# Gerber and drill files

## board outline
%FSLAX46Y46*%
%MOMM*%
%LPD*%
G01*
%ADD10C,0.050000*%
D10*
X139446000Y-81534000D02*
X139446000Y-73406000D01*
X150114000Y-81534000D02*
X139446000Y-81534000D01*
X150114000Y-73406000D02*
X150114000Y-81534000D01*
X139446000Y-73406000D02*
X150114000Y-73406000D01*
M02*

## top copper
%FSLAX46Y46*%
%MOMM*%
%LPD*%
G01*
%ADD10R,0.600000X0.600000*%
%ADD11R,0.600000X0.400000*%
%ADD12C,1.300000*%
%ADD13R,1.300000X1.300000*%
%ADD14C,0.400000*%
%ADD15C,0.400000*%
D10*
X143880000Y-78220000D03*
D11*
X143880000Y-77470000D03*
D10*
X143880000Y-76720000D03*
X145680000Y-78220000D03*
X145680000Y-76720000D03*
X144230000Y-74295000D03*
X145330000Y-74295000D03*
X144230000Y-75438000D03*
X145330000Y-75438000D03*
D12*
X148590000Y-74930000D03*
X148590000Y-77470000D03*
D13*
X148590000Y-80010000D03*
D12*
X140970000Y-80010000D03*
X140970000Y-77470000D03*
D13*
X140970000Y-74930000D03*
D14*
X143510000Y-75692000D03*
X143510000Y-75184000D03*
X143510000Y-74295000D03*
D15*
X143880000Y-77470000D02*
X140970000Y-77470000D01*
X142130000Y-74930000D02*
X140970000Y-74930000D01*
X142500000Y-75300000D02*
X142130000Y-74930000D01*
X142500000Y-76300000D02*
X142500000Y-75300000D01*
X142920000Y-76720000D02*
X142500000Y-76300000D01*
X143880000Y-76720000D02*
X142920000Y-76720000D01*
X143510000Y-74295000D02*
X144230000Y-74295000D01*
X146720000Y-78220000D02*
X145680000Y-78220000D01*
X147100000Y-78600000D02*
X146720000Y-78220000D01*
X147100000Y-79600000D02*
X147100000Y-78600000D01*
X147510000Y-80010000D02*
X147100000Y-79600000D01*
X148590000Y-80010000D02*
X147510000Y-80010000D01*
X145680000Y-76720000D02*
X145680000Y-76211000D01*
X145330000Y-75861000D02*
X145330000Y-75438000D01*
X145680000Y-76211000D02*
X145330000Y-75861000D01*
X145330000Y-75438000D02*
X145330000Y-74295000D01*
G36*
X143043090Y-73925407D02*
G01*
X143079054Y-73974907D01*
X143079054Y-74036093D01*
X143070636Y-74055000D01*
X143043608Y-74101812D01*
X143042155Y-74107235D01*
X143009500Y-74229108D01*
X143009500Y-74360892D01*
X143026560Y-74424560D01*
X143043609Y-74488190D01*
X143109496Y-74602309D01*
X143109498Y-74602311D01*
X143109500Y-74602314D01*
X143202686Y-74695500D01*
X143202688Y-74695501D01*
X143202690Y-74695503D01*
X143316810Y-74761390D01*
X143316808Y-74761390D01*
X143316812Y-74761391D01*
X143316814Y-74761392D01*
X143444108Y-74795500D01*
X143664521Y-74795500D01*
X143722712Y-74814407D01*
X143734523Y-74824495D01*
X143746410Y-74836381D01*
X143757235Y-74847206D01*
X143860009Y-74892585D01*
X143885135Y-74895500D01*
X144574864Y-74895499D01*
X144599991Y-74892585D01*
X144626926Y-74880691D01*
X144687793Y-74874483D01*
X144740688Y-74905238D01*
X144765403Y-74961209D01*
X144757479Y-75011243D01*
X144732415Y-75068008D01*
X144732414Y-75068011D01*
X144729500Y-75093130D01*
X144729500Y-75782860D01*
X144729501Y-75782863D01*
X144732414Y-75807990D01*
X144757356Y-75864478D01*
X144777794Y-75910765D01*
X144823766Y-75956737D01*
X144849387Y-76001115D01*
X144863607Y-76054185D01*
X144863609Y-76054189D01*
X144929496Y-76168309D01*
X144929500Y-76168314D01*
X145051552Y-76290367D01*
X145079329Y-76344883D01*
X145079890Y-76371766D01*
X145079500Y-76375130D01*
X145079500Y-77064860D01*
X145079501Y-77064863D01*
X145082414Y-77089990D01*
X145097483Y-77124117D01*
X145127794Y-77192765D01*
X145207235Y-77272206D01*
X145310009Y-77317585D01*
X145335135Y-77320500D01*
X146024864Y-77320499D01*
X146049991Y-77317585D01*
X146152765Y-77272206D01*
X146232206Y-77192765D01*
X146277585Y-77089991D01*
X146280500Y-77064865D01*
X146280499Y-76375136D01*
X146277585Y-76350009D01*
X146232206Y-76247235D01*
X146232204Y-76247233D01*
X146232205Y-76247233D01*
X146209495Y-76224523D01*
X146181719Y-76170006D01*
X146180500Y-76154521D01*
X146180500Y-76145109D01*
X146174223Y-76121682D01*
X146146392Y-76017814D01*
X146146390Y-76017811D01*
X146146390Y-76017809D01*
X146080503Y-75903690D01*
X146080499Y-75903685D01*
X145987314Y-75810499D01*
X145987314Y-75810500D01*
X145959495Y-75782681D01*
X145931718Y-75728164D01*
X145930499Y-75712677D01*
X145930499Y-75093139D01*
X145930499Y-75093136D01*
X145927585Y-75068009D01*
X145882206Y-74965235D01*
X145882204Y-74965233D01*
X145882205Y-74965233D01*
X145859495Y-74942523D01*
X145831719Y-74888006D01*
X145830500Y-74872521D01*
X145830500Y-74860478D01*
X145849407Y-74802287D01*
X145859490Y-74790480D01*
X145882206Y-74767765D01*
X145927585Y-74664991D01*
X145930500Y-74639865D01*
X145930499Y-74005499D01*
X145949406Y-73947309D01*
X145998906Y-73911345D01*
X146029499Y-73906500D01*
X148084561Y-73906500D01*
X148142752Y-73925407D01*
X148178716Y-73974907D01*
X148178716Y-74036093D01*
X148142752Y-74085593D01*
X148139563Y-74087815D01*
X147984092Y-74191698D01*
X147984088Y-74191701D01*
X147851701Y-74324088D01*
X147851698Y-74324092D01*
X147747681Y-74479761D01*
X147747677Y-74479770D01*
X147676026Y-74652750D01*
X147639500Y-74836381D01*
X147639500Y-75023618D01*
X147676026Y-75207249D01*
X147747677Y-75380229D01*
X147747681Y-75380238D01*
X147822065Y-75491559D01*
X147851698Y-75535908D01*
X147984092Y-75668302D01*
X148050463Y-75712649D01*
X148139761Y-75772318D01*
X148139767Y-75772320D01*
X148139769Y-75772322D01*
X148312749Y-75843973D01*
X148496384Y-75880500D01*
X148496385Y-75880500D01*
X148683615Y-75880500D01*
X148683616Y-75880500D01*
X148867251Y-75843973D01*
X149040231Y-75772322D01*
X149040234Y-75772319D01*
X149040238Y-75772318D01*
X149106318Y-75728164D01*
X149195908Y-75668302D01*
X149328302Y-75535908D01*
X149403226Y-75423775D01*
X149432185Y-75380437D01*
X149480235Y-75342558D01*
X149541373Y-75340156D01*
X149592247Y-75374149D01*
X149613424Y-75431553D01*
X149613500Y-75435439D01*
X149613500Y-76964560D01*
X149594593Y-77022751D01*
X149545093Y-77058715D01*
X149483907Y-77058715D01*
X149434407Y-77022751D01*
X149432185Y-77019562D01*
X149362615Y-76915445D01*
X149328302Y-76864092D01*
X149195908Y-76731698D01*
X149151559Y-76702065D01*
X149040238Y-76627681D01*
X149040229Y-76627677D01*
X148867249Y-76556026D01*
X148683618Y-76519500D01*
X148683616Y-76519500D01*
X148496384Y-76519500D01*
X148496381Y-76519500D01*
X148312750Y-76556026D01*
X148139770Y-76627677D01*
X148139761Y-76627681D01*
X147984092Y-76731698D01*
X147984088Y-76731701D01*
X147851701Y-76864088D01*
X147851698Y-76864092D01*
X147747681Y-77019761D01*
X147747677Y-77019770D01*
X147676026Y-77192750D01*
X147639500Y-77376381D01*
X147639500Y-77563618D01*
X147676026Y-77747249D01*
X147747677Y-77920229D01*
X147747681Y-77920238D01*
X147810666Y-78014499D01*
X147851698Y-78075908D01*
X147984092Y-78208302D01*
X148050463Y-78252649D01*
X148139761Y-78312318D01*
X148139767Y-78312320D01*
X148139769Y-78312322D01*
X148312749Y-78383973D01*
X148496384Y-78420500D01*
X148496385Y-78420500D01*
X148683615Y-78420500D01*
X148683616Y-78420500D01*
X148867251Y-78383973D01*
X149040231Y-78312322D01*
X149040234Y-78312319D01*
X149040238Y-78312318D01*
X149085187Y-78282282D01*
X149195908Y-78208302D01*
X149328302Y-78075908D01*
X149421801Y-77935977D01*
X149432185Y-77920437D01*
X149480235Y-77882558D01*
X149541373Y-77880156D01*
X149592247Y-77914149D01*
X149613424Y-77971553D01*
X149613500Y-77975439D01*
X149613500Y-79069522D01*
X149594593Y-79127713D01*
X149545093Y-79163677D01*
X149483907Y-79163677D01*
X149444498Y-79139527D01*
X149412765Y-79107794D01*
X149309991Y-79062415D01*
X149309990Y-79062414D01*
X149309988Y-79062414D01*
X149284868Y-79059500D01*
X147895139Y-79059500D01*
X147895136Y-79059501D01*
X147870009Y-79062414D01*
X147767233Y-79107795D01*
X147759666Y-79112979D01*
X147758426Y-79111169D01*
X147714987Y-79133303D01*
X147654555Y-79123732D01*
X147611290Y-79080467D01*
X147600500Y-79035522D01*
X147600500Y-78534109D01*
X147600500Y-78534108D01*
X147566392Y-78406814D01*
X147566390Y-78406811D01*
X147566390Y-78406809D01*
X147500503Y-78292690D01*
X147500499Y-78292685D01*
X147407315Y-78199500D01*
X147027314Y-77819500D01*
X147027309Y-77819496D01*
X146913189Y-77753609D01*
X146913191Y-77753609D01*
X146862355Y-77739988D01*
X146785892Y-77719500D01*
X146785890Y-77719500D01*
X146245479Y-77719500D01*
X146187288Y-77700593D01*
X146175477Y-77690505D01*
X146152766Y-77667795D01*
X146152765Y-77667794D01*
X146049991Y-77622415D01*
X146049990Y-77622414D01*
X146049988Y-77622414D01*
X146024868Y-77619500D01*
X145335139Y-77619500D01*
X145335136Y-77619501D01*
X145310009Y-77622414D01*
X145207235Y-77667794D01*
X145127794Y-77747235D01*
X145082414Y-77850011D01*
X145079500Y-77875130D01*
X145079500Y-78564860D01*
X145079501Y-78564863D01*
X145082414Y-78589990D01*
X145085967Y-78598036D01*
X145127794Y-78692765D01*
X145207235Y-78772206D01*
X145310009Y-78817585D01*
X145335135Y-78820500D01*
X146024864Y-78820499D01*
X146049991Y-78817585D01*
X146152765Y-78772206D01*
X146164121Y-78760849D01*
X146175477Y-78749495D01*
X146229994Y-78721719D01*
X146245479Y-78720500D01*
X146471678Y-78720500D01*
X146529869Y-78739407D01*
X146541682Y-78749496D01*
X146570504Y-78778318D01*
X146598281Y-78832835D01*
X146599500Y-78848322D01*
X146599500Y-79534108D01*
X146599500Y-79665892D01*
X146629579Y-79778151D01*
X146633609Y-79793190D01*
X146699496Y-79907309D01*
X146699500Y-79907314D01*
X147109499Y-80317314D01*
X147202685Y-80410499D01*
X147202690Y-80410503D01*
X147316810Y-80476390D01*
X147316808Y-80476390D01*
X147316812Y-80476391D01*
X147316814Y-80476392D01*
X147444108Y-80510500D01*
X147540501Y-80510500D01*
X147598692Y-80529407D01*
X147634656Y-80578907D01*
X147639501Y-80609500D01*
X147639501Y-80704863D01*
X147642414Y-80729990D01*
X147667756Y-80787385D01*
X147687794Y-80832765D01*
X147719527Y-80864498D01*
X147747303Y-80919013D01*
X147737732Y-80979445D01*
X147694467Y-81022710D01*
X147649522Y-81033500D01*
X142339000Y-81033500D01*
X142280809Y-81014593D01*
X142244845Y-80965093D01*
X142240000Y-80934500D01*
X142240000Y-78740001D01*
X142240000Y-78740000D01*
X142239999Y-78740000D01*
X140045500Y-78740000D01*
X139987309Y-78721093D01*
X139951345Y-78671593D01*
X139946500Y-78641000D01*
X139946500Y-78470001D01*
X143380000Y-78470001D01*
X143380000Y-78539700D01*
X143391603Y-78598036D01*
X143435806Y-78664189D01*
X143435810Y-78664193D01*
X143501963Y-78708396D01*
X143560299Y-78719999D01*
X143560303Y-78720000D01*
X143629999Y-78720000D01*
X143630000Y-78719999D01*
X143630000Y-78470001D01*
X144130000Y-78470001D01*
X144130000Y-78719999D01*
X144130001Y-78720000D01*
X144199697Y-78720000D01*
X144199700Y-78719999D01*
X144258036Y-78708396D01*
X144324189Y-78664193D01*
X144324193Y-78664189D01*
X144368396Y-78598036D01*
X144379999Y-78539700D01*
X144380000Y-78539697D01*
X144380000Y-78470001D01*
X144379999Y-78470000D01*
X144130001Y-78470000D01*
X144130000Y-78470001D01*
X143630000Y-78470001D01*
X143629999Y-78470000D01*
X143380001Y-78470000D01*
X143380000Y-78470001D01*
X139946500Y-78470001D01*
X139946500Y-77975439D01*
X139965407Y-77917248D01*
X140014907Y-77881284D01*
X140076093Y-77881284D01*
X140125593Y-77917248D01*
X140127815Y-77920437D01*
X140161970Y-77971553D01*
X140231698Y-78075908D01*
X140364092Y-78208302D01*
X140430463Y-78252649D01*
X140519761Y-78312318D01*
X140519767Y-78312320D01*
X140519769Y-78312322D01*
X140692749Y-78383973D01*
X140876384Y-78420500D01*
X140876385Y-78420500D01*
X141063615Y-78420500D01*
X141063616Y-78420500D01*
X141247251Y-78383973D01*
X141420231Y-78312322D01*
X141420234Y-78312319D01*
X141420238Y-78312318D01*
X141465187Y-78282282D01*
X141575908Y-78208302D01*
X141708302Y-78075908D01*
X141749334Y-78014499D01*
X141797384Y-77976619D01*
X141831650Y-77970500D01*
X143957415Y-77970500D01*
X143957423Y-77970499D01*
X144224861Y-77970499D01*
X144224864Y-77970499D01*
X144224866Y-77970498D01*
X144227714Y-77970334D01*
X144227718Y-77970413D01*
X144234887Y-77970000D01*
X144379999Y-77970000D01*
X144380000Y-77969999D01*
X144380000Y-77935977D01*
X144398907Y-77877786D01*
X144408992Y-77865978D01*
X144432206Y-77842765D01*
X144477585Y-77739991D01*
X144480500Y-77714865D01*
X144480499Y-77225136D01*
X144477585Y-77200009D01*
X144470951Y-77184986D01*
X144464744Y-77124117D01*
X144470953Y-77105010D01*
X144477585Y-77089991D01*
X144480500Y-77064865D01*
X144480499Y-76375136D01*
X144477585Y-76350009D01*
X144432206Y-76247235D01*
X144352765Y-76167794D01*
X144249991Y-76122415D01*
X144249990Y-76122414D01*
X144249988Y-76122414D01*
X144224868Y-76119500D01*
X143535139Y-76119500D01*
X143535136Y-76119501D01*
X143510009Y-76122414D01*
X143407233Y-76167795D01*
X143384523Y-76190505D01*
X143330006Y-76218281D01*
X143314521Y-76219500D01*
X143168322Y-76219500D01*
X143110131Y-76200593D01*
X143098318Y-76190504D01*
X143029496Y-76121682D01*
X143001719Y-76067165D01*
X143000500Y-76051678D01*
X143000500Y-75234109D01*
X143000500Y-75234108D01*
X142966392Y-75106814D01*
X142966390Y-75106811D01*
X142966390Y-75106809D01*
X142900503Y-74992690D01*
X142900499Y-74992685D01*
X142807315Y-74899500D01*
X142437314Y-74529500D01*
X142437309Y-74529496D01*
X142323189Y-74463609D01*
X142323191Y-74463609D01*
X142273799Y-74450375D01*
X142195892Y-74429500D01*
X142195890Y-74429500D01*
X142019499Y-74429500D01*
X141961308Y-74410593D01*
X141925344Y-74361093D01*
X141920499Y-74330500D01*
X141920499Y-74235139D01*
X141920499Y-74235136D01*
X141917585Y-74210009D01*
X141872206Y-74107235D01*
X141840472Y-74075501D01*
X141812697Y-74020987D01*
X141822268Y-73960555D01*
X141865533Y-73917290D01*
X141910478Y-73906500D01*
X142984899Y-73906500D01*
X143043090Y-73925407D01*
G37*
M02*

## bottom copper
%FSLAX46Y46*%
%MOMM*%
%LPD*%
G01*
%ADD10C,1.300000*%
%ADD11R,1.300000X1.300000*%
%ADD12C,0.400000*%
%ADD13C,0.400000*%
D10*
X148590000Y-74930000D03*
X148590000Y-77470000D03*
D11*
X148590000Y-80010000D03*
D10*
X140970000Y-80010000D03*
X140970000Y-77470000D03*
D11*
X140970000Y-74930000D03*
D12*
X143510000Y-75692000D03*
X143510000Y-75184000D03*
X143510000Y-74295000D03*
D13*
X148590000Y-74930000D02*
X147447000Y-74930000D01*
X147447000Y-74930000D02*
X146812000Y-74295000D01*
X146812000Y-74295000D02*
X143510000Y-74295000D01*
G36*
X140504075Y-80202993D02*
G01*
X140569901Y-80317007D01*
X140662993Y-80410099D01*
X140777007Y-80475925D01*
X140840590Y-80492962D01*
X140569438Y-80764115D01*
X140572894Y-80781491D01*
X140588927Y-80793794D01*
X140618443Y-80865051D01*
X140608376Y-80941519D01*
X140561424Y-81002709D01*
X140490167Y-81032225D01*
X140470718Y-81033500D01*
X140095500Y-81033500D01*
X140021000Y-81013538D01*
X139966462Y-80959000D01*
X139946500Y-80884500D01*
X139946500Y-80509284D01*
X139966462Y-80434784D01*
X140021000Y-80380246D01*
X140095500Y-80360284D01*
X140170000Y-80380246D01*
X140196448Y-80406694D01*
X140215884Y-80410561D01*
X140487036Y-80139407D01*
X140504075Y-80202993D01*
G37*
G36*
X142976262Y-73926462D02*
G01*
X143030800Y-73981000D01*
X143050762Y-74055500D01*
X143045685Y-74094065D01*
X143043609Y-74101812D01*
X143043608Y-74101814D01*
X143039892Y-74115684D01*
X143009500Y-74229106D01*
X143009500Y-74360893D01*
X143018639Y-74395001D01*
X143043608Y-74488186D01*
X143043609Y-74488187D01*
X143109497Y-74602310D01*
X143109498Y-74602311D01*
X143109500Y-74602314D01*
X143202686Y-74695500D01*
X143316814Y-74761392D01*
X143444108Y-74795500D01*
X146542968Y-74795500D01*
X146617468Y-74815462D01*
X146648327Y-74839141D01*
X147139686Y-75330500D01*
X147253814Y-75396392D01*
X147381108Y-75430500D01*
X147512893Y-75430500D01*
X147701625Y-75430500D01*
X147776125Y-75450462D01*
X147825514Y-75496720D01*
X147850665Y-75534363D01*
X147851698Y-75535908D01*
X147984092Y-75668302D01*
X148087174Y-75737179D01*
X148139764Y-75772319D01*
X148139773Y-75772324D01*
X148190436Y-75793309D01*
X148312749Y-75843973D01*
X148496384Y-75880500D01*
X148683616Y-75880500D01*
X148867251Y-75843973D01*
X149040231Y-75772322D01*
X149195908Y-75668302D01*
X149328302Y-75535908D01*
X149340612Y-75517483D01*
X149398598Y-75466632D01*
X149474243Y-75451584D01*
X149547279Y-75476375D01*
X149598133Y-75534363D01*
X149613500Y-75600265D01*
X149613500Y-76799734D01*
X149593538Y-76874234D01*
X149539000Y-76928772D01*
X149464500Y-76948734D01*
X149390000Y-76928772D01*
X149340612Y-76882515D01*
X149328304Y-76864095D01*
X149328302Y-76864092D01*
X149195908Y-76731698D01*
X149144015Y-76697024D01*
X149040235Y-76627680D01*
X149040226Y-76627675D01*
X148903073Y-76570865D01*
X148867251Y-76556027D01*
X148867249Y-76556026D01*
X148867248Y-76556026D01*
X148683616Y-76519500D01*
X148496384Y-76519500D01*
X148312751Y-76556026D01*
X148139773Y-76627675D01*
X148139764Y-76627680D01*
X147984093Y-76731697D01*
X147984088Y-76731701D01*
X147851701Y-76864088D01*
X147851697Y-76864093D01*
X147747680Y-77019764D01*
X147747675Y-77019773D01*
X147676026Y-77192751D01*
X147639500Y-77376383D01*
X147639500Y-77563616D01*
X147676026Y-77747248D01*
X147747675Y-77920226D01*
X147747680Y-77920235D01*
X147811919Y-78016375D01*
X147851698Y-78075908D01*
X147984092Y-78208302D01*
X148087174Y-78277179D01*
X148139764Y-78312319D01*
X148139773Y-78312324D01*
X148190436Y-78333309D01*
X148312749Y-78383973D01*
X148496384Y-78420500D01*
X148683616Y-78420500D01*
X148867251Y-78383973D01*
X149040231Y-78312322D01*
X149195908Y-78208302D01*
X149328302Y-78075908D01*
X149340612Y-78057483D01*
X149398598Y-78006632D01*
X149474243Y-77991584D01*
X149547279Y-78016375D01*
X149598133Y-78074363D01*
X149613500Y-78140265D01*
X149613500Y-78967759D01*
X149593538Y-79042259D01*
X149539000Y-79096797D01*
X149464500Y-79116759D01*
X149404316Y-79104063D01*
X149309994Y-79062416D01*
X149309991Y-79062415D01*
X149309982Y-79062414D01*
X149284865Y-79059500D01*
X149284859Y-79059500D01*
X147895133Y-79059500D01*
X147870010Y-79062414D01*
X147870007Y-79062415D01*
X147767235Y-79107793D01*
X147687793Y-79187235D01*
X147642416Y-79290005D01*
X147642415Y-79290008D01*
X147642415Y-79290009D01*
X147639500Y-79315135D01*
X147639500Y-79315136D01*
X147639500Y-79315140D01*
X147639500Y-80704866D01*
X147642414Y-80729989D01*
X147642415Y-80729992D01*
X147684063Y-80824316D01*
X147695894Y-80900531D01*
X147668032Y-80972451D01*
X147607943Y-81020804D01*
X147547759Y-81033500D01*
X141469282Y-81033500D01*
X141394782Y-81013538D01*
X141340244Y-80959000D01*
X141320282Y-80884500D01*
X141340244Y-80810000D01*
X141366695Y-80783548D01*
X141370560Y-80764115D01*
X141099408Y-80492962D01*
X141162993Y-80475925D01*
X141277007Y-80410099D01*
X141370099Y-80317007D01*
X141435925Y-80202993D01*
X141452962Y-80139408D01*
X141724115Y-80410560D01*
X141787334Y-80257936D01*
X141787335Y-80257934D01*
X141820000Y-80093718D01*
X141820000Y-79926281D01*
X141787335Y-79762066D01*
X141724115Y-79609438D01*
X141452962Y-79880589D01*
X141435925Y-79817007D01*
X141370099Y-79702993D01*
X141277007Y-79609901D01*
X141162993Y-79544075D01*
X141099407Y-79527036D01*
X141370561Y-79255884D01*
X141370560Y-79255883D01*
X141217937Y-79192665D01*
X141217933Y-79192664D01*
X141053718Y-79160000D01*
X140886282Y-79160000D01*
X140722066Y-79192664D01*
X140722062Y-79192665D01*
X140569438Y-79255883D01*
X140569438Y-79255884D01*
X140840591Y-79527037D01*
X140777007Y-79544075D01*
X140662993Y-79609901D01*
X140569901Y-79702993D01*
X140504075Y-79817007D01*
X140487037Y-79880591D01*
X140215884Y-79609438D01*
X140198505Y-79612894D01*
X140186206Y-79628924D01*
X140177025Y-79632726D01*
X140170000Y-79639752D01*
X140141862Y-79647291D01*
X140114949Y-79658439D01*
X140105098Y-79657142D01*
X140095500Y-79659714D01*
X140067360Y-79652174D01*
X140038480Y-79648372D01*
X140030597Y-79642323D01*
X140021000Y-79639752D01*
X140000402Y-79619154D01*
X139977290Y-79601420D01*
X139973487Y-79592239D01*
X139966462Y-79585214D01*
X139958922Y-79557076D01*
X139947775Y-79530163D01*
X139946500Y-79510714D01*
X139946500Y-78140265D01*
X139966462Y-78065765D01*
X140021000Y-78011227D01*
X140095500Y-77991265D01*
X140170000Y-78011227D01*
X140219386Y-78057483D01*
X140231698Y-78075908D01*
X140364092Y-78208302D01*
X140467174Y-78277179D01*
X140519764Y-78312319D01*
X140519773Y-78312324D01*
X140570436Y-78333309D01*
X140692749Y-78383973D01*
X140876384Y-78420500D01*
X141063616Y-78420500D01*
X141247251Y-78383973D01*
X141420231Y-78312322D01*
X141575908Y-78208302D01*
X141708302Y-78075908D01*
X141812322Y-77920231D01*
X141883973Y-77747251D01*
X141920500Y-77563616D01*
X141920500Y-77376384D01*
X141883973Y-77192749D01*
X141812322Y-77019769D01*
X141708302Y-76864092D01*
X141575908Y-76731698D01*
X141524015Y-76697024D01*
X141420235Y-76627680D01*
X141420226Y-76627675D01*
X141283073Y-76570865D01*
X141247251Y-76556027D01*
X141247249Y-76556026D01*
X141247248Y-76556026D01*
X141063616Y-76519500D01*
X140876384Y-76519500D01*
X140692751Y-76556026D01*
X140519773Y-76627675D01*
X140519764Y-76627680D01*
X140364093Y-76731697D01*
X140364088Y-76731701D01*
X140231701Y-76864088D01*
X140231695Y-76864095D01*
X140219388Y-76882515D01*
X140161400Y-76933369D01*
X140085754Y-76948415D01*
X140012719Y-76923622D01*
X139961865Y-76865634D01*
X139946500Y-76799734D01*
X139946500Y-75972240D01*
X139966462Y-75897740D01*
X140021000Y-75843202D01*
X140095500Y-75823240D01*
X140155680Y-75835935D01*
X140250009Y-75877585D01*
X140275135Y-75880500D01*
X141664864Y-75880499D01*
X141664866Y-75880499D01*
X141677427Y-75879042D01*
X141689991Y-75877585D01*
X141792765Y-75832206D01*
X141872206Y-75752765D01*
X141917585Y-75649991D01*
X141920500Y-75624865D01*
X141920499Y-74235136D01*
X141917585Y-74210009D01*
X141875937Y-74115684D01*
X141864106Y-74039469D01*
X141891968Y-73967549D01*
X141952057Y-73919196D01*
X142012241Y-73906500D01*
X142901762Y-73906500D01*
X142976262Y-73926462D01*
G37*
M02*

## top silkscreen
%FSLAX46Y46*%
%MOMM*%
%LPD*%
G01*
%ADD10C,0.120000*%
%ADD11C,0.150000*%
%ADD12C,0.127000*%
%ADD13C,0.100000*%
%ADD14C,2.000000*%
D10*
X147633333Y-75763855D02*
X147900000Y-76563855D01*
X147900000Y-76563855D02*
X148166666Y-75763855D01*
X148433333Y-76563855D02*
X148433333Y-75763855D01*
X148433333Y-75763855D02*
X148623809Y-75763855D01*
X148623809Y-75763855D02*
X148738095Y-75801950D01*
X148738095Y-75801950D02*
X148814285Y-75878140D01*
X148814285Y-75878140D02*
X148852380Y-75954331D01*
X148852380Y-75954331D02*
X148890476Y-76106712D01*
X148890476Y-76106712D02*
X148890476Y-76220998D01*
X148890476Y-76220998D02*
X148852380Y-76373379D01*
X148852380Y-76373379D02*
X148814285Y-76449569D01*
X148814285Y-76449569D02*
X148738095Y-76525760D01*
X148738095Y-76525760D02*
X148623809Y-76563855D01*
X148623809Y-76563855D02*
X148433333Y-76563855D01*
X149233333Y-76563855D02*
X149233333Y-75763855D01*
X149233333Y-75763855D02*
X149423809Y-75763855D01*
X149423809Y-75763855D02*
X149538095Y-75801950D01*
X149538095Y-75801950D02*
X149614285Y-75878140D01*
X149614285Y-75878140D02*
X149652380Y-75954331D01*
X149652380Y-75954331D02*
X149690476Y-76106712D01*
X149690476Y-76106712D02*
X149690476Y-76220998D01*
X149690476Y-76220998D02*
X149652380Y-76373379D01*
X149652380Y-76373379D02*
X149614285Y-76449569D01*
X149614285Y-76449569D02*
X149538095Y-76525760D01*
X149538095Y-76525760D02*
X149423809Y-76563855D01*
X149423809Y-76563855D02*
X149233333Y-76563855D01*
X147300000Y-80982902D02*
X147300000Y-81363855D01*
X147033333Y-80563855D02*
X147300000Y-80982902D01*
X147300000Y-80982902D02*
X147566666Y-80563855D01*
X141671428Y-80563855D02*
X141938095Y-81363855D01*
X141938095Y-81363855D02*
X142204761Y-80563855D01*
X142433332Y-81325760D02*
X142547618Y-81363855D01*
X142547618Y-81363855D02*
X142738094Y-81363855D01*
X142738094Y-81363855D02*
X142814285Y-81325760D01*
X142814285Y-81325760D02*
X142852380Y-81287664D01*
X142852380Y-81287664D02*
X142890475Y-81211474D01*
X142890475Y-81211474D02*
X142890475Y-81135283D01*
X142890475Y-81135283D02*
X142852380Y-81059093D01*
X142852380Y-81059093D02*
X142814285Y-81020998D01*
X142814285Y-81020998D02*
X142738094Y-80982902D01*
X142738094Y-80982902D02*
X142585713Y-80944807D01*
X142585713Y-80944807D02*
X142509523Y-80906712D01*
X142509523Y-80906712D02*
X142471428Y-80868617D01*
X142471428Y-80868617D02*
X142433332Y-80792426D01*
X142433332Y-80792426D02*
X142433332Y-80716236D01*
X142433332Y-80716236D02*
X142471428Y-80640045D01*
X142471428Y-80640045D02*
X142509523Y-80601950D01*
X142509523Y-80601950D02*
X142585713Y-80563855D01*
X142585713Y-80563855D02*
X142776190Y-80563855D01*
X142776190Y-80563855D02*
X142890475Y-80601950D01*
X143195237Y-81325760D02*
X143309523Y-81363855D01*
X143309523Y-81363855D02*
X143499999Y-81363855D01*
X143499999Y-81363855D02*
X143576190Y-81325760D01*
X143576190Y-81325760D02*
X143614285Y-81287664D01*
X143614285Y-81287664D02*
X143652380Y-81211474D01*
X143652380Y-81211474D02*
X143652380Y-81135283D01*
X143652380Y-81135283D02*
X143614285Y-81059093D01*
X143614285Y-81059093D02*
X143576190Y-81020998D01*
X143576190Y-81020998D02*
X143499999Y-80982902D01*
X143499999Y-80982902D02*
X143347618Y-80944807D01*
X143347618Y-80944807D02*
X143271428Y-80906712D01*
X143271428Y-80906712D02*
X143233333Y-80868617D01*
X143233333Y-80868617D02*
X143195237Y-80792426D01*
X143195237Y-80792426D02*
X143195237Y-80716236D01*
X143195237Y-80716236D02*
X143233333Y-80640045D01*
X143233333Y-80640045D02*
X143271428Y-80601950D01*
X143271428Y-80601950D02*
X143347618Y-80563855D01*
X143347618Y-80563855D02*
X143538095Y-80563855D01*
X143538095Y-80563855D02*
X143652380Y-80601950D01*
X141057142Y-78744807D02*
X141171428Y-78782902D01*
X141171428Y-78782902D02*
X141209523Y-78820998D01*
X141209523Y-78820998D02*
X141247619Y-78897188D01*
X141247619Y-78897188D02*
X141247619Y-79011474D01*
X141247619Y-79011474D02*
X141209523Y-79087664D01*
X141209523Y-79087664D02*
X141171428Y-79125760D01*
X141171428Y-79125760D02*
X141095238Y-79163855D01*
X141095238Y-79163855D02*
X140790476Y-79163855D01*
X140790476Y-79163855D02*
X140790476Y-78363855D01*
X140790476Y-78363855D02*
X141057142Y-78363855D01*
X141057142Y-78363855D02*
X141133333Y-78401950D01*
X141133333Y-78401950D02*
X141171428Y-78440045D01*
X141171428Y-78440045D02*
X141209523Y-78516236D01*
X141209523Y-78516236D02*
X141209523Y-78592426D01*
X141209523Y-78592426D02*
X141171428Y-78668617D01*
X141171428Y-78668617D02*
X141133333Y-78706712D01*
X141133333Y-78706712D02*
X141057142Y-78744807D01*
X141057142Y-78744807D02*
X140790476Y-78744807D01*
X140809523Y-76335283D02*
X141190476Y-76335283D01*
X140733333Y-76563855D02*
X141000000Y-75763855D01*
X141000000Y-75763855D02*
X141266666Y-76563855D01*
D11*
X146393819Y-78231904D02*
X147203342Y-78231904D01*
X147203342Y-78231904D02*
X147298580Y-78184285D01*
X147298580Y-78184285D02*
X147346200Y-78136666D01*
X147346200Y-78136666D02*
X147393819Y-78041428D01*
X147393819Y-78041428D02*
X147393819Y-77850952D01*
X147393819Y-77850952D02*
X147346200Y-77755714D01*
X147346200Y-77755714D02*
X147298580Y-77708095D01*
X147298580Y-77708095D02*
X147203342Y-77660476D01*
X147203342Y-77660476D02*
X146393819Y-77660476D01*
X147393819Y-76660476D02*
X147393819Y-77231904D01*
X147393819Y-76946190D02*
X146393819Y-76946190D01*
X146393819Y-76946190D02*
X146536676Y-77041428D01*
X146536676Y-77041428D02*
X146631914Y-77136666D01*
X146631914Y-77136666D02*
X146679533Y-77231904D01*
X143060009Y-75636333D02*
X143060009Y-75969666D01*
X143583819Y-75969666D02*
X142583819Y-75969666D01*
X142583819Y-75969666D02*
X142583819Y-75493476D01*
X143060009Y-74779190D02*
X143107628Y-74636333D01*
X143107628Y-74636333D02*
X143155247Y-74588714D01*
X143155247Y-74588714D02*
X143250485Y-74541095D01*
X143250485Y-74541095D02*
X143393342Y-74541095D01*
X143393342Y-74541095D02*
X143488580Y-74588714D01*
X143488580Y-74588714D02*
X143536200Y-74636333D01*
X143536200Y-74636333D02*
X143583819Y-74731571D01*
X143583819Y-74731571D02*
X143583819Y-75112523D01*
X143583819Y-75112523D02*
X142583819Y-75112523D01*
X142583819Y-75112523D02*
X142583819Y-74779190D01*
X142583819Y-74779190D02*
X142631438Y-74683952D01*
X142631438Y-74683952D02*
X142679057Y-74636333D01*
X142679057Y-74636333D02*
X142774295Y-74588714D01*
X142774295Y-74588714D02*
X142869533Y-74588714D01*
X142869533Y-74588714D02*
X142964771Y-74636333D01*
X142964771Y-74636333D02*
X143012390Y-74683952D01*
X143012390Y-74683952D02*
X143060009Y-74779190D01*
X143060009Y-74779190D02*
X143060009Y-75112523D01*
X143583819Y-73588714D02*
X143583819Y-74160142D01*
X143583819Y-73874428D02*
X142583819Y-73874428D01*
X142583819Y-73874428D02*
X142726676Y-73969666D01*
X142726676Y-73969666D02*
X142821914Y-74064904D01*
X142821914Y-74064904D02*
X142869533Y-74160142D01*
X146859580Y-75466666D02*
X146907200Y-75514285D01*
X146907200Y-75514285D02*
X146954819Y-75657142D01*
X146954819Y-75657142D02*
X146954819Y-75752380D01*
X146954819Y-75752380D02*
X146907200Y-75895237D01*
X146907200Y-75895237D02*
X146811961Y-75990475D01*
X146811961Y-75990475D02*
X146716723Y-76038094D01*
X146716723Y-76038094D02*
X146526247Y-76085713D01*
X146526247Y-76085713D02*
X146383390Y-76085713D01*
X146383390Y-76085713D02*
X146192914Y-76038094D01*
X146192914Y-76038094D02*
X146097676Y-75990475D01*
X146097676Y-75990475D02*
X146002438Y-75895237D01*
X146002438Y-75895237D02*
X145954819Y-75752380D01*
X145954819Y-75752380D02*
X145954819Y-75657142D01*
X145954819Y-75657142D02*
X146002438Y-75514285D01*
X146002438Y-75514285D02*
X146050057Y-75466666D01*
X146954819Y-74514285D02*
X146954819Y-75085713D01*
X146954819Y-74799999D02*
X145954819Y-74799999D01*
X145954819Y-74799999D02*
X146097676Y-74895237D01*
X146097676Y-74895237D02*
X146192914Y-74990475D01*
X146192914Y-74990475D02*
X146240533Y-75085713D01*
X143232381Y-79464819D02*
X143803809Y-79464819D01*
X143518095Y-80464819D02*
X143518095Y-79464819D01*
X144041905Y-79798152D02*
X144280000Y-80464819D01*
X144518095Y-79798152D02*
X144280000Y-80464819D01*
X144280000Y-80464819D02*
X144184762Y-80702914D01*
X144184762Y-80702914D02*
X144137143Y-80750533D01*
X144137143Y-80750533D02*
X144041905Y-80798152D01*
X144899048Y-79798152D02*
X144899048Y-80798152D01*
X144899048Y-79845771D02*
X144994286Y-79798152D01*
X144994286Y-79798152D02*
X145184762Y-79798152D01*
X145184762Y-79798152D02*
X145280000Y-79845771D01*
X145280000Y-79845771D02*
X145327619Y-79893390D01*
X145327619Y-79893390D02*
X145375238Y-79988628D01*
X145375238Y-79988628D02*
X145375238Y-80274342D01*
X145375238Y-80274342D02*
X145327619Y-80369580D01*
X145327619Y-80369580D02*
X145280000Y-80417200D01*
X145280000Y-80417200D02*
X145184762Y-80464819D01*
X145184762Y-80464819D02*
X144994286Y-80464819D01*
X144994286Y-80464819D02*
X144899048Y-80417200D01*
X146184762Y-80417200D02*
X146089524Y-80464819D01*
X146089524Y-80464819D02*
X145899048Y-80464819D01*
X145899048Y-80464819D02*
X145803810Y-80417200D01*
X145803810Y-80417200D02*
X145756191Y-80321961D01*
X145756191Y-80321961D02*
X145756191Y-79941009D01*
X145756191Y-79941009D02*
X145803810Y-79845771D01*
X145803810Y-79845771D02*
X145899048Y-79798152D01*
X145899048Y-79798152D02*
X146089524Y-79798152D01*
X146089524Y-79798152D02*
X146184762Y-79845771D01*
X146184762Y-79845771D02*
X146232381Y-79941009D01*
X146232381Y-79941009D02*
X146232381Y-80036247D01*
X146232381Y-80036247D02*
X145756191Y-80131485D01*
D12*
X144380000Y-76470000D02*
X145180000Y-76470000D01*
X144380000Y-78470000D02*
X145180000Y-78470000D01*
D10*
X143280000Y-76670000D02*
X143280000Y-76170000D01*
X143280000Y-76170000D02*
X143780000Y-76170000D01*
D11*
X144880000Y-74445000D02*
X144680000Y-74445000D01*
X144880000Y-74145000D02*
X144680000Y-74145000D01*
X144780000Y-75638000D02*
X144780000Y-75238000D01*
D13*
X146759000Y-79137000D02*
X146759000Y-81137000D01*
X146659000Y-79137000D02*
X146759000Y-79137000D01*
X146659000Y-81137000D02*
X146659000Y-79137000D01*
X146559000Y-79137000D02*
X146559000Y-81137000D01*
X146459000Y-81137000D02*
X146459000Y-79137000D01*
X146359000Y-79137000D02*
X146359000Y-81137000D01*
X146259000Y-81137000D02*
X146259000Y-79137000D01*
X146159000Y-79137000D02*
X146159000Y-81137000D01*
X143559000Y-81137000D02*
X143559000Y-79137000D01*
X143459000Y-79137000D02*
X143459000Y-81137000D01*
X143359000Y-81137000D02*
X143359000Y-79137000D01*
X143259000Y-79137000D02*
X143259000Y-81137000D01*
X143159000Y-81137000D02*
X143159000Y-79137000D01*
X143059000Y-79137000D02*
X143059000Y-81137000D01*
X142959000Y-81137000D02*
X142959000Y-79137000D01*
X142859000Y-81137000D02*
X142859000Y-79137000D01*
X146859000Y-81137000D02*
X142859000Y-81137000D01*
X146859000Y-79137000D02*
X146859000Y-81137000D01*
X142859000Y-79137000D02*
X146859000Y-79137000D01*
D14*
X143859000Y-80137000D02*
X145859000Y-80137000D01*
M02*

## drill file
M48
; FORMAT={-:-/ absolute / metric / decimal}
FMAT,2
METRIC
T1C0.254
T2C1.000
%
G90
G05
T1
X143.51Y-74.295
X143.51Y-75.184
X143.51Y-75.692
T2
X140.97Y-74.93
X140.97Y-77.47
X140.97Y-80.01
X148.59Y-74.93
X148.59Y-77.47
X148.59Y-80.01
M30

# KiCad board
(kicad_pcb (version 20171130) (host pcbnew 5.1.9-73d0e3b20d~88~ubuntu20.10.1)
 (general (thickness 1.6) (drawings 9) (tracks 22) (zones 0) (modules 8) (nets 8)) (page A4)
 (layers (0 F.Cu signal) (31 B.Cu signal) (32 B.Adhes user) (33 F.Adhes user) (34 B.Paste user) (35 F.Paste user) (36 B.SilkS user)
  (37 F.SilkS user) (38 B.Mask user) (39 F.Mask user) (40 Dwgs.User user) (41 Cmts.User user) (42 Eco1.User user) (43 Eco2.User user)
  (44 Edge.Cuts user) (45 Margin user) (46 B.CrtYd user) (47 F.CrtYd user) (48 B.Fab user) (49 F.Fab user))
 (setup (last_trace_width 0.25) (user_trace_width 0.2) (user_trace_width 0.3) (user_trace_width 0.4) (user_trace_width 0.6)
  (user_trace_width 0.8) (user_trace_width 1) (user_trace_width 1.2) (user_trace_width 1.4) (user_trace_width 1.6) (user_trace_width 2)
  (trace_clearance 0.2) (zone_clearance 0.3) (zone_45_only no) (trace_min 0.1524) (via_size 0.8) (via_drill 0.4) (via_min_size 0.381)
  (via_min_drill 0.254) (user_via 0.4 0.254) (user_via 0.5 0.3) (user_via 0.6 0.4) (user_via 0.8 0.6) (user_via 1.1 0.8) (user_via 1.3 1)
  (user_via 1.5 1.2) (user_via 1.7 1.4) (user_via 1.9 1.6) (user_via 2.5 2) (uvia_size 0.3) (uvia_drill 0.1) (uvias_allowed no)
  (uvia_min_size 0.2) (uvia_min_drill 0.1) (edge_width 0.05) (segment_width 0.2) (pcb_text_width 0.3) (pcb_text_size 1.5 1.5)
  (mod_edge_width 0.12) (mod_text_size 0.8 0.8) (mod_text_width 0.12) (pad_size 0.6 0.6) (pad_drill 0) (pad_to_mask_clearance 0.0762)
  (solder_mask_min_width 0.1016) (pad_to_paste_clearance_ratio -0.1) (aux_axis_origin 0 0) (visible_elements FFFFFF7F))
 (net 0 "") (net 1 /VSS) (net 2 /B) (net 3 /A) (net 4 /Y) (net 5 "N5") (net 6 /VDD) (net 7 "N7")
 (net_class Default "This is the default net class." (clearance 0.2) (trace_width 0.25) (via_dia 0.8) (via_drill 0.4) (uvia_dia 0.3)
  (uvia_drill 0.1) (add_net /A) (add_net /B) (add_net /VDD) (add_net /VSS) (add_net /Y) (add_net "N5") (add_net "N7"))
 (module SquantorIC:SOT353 (layer F.Cu) (at 144.78 77.47 270)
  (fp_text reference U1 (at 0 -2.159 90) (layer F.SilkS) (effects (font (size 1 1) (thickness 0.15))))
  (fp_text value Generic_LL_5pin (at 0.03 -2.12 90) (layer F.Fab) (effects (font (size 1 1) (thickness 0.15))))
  (fp_line (start -1 0.4) (end -1 -0.4) (layer F.SilkS) (width 0.127))
  (fp_line (start 1 0.4) (end 1 -0.4) (layer F.SilkS) (width 0.127))
  (fp_line (start -0.8 1.5) (end -1.3 1.5) (layer F.SilkS) (width 0.12))
  (fp_line (start -1.3 1.5) (end -1.3 1) (layer F.SilkS) (width 0.12))
  (pad 3 smd rect (at 0.75 0.9 270) (size 0.6 0.6) (layers F.Cu F.Paste F.Mask) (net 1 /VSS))
  (pad 2 smd rect (at 0 0.9 270) (size 0.4 0.6) (layers F.Cu F.Paste F.Mask) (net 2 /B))
  (pad 1 smd rect (at -0.75 0.9 270) (size 0.6 0.6) (layers F.Cu F.Paste F.Mask) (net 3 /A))
  (pad 4 smd rect (at 0.75 -0.9 270) (size 0.6 0.6) (layers F.Cu F.Paste F.Mask) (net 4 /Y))
  (pad 5 smd rect (at -0.75 -0.9 270) (size 0.6 0.6) (layers F.Cu F.Paste F.Mask) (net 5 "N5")))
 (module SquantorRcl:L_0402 (layer F.Cu) (at 144.78 74.295 180)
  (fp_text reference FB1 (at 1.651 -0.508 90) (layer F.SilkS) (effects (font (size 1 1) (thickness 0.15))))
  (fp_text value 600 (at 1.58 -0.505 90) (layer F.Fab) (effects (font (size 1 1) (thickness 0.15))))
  (fp_line (start -0.1 -0.15) (end 0.1 -0.15) (layer F.SilkS) (width 0.15))
  (fp_line (start -0.1 0.15) (end 0.1 0.15) (layer F.SilkS) (width 0.15))
  (pad 2 smd rect (at 0.55 0 180) (size 0.6 0.6) (layers F.Cu F.Paste F.Mask) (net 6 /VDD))
  (pad 1 smd rect (at -0.55 0 180) (size 0.6 0.6) (layers F.Cu F.Paste F.Mask) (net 5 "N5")))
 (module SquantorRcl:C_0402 (layer F.Cu) (at 144.78 75.438 180)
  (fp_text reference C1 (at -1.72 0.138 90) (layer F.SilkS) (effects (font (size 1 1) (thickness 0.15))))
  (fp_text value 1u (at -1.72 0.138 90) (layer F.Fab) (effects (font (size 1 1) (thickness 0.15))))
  (fp_line (start 0 -0.2) (end 0 0.2) (layer F.SilkS) (width 0.15))
  (pad 2 smd rect (at 0.55 0 180) (size 0.6 0.6) (layers F.Cu F.Paste F.Mask) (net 1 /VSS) (zone_connect 2))
  (pad 1 smd rect (at -0.55 0 180) (size 0.6 0.6) (layers F.Cu F.Paste F.Mask) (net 5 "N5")))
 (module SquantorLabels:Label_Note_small (layer F.Cu) (at 141.859 80.137)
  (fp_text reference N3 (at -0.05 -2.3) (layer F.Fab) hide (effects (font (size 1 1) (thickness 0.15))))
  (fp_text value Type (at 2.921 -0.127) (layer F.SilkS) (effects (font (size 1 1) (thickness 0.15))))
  (fp_line (start 4.9 -1) (end 4.9 1) (layer F.SilkS) (width 0.1))
  (fp_line (start 4.8 -1) (end 4.9 -1) (layer F.SilkS) (width 0.1))
  (fp_line (start 4.8 1) (end 4.8 -1) (layer F.SilkS) (width 0.1))
  (fp_line (start 4.7 -1) (end 4.7 1) (layer F.SilkS) (width 0.1))
  (fp_line (start 4.6 1) (end 4.6 -1) (layer F.SilkS) (width 0.1))
  (fp_line (start 4.5 -1) (end 4.5 1) (layer F.SilkS) (width 0.1))
  (fp_line (start 4.4 1) (end 4.4 -1) (layer F.SilkS) (width 0.1))
  (fp_line (start 4.3 -1) (end 4.3 1) (layer F.SilkS) (width 0.1))
  (fp_line (start 1.7 1) (end 1.7 -1) (layer F.SilkS) (width 0.1))
  (fp_line (start 1.6 -1) (end 1.6 1) (layer F.SilkS) (width 0.1))
  (fp_line (start 1.5 1) (end 1.5 -1) (layer F.SilkS) (width 0.1))
  (fp_line (start 1.4 -1) (end 1.4 1) (layer F.SilkS) (width 0.1))
  (fp_line (start 1.3 1) (end 1.3 -1) (layer F.SilkS) (width 0.1))
  (fp_line (start 1.2 -1) (end 1.2 1) (layer F.SilkS) (width 0.1))
  (fp_line (start 1.1 1) (end 1.1 -1) (layer F.SilkS) (width 0.1)) (fp_line (start 1 1) (end 1 -1) (layer F.SilkS) (width 0.1))
  (fp_line (start 5 1) (end 1 1) (layer F.SilkS) (width 0.1)) (fp_line (start 5 -1) (end 5 1) (layer F.SilkS) (width 0.1))
  (fp_line (start 1 -1) (end 5 -1) (layer F.SilkS) (width 0.1)) (fp_line (start 2 0) (end 4 0) (layer F.SilkS) (width 2)))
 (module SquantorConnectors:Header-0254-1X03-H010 (layer B.Cu) (at 148.59 77.47 90)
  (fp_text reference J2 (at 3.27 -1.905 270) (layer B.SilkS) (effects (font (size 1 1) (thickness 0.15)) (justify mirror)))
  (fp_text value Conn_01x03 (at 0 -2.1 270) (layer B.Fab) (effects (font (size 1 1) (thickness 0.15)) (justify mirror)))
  (pad 3 thru_hole circle (at 2.54 0 270) (size 1.3 1.3) (drill 1) (layers *.Cu *.Mask) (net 6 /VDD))
  (pad 2 thru_hole circle (at 0 0 270) (size 1.3 1.3) (drill 1) (layers *.Cu *.Mask) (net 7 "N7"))
  (pad 1 thru_hole rect (at -2.54 0 270) (size 1.3 1.3) (drill 1) (layers *.Cu *.Mask) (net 4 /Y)))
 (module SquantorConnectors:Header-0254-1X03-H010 (layer B.Cu) (at 140.97 77.47 270)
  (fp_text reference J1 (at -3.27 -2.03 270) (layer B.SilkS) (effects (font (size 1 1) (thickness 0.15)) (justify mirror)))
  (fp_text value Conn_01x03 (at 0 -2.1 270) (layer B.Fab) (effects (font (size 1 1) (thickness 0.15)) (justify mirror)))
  (pad 3 thru_hole circle (at 2.54 0 90) (size 1.3 1.3) (drill 1) (layers *.Cu *.Mask) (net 1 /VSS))
  (pad 2 thru_hole circle (at 0 0 90) (size 1.3 1.3) (drill 1) (layers *.Cu *.Mask) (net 2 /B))
  (pad 1 thru_hole rect (at -2.54 0 90) (size 1.3 1.3) (drill 1) (layers *.Cu *.Mask) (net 3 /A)))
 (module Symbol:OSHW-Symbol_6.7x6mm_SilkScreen (layer B.Cu) (at 144.7 77.2 180)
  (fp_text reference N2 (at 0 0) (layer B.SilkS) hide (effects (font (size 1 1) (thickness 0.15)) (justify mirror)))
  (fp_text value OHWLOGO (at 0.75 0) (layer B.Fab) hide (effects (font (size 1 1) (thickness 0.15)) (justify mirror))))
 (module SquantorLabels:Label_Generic (layer B.Cu) (at 145.491 81 180)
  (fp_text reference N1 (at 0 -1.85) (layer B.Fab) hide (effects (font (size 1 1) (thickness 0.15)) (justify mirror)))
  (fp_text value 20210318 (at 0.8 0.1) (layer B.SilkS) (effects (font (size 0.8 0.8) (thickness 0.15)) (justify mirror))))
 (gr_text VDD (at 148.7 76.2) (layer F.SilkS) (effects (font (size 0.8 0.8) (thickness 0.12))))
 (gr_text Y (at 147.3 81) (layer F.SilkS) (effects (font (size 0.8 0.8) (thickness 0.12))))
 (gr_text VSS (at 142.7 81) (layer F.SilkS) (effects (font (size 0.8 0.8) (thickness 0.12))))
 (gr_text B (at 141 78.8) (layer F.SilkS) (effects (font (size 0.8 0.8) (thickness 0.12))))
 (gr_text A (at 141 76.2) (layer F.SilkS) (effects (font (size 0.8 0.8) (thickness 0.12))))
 (gr_line (start 139.446 81.534) (end 139.446 73.406) (layer Edge.Cuts) (width 0.05))
 (gr_line (start 150.114 81.534) (end 139.446 81.534) (layer Edge.Cuts) (width 0.05))
 (gr_line (start 150.114 73.406) (end 150.114 81.534) (layer Edge.Cuts) (width 0.05))
 (gr_line (start 139.446 73.406) (end 150.114 73.406) (layer Edge.Cuts) (width 0.05))
 (via (at 143.51 75.692) (size 0.4) (drill 0.254) (layers F.Cu B.Cu) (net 1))
 (via (at 143.51 75.184) (size 0.4) (drill 0.254) (layers F.Cu B.Cu) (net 1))
 (segment (start 143.88 77.47) (end 140.97 77.47) (width 0.4) (layer F.Cu) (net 2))
 (segment (start 142.13 74.93) (end 140.97 74.93) (width 0.4) (layer F.Cu) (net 3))
 (segment (start 142.5 75.3) (end 142.13 74.93) (width 0.4) (layer F.Cu) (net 3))
 (segment (start 142.5 76.3) (end 142.5 75.3) (width 0.4) (layer F.Cu) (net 3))
 (segment (start 142.92 76.72) (end 142.5 76.3) (width 0.4) (layer F.Cu) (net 3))
 (segment (start 143.88 76.72) (end 142.92 76.72) (width 0.4) (layer F.Cu) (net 3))
 (segment (start 148.59 74.93) (end 147.447 74.93) (width 0.4) (layer B.Cu) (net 6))
 (segment (start 147.447 74.93) (end 146.812 74.295) (width 0.4) (layer B.Cu) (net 6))
 (via (at 143.51 74.295) (size 0.4) (drill 0.254) (layers F.Cu B.Cu) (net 6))
 (segment (start 146.812 74.295) (end 143.51 74.295) (width 0.4) (layer B.Cu) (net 6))
 (segment (start 143.51 74.295) (end 144.23 74.295) (width 0.4) (layer F.Cu) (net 6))
 (segment (start 146.72 78.22) (end 145.68 78.22) (width 0.4) (layer F.Cu) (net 4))
 (segment (start 147.1 78.6) (end 146.72 78.22) (width 0.4) (layer F.Cu) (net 4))
 (segment (start 147.1 79.6) (end 147.1 78.6) (width 0.4) (layer F.Cu) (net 4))
 (segment (start 147.51 80.01) (end 147.1 79.6) (width 0.4) (layer F.Cu) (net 4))
 (segment (start 148.59 80.01) (end 147.51 80.01) (width 0.4) (layer F.Cu) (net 4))
 (segment (start 145.68 76.72) (end 145.68 76.211) (width 0.4) (layer F.Cu) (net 5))
 (segment (start 145.33 75.861) (end 145.33 75.438) (width 0.4) (layer F.Cu) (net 5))
 (segment (start 145.68 76.211) (end 145.33 75.861) (width 0.4) (layer F.Cu) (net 5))
 (segment (start 145.33 75.438) (end 145.33 74.295) (width 0.4) (layer F.Cu) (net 5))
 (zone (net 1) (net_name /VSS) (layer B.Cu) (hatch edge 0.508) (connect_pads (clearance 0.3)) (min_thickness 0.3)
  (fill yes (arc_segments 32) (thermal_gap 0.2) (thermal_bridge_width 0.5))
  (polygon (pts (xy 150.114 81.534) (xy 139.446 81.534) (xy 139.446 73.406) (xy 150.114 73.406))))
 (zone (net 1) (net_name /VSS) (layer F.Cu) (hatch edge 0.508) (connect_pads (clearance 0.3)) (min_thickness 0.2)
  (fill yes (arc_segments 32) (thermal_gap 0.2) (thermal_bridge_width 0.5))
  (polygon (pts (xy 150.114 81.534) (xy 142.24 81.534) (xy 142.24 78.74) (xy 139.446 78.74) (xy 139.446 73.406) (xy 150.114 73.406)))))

